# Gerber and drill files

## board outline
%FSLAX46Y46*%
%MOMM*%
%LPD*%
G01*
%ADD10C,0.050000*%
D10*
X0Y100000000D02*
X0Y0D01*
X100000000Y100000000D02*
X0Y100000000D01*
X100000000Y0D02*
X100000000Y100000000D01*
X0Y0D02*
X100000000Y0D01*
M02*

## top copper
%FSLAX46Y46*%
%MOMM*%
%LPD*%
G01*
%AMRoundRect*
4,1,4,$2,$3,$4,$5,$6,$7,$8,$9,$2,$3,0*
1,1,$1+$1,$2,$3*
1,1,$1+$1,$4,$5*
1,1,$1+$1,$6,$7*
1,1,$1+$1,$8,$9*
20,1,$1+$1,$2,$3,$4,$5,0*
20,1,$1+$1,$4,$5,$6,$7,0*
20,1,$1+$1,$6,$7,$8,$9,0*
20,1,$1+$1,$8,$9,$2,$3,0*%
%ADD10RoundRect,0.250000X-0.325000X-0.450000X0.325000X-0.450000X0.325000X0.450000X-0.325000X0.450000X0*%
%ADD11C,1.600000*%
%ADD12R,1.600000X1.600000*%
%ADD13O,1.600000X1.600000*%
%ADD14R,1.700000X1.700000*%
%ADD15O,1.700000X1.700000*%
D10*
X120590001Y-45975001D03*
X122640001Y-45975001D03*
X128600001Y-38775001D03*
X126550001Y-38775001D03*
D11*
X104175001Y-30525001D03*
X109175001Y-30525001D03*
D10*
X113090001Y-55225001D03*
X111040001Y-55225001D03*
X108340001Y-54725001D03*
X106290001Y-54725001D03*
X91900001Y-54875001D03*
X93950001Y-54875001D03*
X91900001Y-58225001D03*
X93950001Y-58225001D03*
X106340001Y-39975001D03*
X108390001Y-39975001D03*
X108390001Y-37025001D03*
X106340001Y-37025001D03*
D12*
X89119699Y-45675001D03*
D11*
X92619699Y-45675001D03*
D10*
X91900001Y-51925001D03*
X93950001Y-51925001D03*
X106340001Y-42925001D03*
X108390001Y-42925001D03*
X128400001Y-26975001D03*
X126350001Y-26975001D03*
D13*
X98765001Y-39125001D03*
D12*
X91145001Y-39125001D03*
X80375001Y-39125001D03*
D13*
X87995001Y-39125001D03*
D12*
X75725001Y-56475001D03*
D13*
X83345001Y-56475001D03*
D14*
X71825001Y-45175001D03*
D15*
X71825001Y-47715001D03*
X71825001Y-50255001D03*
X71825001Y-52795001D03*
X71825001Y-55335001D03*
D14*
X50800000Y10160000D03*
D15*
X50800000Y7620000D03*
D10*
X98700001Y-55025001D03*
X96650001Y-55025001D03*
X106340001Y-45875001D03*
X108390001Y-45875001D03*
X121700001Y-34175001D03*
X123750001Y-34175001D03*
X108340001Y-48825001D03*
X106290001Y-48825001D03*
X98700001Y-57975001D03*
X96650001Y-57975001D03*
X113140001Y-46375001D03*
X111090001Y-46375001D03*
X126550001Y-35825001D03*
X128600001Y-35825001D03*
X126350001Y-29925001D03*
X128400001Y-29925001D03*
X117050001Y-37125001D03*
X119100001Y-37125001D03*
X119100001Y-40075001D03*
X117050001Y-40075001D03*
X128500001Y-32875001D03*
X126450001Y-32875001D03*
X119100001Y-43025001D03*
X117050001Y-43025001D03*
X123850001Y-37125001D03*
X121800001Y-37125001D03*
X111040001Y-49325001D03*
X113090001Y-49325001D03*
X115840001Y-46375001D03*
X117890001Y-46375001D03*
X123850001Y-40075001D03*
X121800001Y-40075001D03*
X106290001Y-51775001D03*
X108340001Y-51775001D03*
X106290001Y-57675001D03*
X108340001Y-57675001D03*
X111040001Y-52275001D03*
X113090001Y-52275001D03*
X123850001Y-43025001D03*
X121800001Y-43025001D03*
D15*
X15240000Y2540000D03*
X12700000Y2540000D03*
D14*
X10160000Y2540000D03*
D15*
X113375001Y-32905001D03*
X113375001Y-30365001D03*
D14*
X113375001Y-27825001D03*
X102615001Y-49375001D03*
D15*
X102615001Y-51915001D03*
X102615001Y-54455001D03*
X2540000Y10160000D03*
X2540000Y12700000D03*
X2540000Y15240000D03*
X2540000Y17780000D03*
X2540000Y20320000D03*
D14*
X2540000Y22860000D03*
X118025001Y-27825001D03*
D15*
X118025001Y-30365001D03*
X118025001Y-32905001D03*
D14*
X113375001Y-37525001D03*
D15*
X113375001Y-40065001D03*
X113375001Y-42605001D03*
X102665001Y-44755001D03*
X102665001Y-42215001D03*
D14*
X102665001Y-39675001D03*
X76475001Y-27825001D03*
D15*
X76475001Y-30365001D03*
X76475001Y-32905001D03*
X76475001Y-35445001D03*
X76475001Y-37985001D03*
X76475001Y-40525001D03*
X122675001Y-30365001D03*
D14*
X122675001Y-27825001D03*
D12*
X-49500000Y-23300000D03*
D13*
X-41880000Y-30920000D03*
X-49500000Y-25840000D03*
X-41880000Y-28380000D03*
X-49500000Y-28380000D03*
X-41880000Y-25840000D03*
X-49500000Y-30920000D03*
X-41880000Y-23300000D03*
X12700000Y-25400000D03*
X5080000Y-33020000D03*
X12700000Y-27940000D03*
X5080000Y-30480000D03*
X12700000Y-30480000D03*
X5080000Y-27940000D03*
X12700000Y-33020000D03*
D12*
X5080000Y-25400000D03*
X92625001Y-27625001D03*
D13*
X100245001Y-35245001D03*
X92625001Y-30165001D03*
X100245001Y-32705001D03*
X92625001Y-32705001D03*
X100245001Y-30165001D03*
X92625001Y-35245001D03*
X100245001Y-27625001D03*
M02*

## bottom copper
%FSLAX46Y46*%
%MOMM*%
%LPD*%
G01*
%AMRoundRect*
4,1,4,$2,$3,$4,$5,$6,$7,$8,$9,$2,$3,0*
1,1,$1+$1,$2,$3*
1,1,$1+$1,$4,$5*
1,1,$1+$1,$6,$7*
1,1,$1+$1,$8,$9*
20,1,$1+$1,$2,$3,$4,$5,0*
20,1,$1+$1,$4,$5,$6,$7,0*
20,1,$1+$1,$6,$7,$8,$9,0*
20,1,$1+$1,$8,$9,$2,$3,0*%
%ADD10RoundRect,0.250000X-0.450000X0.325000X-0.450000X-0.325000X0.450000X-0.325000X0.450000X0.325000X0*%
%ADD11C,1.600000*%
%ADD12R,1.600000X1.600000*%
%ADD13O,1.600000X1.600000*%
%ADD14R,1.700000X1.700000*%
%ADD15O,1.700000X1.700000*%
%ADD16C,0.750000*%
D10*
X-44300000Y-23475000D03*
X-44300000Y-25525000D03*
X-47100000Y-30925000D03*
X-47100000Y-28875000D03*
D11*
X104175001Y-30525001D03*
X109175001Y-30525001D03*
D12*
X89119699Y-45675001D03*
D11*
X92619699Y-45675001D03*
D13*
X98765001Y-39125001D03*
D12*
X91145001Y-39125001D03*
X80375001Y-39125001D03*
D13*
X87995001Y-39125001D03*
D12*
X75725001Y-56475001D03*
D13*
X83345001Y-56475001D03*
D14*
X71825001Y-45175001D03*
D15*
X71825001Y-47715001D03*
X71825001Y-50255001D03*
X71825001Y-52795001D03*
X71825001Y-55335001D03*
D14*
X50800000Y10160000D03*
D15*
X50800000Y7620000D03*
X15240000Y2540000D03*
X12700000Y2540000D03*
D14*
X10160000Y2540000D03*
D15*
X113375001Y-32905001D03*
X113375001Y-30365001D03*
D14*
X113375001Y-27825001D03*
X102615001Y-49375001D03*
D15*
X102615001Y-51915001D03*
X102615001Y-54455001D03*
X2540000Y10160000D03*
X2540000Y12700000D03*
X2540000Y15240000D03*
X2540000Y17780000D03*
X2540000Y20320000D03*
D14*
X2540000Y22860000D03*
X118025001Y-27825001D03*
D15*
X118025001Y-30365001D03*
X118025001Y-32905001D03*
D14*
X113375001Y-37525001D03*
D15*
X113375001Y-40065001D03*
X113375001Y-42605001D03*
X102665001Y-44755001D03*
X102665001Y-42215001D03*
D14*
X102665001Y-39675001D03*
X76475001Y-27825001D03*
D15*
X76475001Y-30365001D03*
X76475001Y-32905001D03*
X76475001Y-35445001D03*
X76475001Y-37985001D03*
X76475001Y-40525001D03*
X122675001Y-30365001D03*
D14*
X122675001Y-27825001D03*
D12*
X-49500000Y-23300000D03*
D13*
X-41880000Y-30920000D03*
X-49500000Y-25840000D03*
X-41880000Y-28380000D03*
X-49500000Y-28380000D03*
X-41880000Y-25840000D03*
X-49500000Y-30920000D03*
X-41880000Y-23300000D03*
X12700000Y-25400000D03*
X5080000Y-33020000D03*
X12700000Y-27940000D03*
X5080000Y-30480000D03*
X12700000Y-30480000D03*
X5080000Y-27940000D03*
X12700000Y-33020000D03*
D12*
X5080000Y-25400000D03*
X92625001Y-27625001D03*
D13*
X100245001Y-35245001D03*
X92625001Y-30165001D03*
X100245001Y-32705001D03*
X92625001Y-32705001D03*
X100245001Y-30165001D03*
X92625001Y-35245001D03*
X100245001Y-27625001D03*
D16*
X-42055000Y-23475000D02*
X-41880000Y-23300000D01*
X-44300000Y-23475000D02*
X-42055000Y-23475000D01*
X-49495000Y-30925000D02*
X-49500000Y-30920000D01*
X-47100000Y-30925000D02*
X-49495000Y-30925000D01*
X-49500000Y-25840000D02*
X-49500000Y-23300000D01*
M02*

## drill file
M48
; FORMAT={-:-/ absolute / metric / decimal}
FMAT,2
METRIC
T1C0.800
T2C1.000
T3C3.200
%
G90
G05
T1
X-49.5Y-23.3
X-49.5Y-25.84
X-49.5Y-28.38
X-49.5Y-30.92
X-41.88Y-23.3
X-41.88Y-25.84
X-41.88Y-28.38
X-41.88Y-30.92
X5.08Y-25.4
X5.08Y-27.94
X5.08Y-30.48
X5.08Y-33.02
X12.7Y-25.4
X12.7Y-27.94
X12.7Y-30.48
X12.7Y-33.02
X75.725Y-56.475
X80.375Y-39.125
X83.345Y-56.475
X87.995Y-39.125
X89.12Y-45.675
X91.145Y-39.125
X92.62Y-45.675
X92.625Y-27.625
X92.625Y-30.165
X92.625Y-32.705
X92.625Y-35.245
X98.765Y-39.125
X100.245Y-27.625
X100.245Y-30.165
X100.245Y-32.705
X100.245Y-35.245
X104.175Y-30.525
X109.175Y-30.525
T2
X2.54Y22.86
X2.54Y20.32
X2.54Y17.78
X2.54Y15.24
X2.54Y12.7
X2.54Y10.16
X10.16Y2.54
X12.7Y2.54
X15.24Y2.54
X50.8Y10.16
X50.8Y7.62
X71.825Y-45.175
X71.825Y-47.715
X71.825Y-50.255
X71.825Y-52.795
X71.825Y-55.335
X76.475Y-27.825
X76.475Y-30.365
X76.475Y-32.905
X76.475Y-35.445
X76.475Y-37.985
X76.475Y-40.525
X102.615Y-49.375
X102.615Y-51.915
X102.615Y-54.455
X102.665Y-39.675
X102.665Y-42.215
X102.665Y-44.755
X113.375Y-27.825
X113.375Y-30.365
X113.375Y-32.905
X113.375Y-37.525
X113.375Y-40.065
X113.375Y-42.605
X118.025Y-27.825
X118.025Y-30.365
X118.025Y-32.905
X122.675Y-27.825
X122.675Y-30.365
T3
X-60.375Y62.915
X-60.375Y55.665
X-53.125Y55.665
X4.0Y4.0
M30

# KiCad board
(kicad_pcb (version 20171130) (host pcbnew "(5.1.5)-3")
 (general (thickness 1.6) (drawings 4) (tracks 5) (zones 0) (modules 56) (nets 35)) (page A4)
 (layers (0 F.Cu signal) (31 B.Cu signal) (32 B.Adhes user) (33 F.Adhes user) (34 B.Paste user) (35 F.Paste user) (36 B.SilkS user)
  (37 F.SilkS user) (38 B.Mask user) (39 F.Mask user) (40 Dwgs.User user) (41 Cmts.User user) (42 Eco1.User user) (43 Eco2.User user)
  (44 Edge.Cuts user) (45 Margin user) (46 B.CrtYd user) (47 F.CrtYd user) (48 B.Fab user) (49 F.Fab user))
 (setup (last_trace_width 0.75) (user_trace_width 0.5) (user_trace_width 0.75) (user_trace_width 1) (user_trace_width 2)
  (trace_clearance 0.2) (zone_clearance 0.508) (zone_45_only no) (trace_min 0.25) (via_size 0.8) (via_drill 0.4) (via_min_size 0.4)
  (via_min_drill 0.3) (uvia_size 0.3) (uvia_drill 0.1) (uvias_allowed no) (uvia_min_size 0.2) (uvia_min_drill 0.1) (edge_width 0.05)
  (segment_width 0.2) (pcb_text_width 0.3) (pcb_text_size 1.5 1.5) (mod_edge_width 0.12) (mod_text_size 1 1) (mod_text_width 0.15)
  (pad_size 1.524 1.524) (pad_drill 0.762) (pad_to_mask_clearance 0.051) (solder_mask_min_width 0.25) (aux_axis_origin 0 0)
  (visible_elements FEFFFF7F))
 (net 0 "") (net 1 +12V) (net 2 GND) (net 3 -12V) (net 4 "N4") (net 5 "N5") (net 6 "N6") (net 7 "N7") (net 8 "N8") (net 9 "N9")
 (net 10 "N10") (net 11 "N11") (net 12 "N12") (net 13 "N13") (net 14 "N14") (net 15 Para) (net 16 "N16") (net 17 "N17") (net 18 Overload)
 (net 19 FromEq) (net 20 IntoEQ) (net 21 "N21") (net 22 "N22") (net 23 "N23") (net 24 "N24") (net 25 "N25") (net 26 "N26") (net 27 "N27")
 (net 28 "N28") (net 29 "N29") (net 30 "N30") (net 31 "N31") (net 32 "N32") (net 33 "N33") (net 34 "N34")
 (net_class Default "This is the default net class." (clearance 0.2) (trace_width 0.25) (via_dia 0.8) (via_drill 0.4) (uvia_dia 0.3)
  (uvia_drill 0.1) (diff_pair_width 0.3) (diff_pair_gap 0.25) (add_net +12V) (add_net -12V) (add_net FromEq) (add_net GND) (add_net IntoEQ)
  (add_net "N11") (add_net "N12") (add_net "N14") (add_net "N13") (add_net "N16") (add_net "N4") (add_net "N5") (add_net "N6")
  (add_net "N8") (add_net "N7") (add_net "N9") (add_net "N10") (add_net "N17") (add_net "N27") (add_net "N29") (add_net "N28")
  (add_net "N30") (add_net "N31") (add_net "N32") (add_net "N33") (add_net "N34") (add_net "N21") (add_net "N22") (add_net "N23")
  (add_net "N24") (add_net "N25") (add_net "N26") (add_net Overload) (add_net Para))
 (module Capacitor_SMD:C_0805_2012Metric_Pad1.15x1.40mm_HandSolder (layer B.Cu) (at -44.3 24.5 270)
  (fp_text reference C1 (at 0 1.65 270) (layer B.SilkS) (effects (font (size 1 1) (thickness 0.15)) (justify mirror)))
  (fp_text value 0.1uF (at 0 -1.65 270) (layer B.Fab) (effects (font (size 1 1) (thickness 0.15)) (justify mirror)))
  (pad 1 smd roundrect (at -1.025 0 270) (size 1.15 1.4) (layers B.Cu B.Paste B.Mask) (roundrect_rratio 0.217391) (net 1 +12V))
  (pad 2 smd roundrect (at 1.025 0 270) (size 1.15 1.4) (layers B.Cu B.Paste B.Mask) (roundrect_rratio 0.217391) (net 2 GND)))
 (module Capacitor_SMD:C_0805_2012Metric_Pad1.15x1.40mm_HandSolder (layer B.Cu) (at -47.1 29.9 270)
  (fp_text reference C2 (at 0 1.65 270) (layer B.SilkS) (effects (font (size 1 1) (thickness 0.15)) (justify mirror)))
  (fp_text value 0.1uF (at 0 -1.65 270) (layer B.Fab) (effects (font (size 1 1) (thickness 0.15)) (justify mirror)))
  (pad 2 smd roundrect (at 1.025 0 270) (size 1.15 1.4) (layers B.Cu B.Paste B.Mask) (roundrect_rratio 0.217391) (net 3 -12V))
  (pad 1 smd roundrect (at -1.025 0 270) (size 1.15 1.4) (layers B.Cu B.Paste B.Mask) (roundrect_rratio 0.217391) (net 2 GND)))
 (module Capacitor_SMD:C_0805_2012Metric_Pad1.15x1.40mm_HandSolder (layer F.Cu) (at 121.615001 45.975001)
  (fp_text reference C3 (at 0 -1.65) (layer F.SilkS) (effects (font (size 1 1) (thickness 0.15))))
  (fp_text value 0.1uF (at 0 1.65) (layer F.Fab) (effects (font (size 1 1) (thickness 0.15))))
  (pad 1 smd roundrect (at -1.025 0) (size 1.15 1.4) (layers F.Cu F.Paste F.Mask) (roundrect_rratio 0.217391) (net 1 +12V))
  (pad 2 smd roundrect (at 1.025 0) (size 1.15 1.4) (layers F.Cu F.Paste F.Mask) (roundrect_rratio 0.217391) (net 2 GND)))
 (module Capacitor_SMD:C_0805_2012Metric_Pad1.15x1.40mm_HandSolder (layer F.Cu) (at 127.575001 38.775001)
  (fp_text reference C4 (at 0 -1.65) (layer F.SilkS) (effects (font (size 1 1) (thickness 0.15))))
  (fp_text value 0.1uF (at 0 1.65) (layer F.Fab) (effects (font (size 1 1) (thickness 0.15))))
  (pad 2 smd roundrect (at 1.025 0) (size 1.15 1.4) (layers F.Cu F.Paste F.Mask) (roundrect_rratio 0.217391) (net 3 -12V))
  (pad 1 smd roundrect (at -1.025 0) (size 1.15 1.4) (layers F.Cu F.Paste F.Mask) (roundrect_rratio 0.217391) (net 2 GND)))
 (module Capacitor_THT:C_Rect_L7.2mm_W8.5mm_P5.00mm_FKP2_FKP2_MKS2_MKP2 (layer F.Cu) (at 104.175001 30.525001)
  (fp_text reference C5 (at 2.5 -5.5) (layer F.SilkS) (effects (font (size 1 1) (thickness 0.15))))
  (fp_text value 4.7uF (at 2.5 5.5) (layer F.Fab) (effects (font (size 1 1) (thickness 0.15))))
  (pad 1 thru_hole circle (at 0 0) (size 1.6 1.6) (drill 0.8) (layers *.Cu *.Mask) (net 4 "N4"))
  (pad 2 thru_hole circle (at 5 0) (size 1.6 1.6) (drill 0.8) (layers *.Cu *.Mask) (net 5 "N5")))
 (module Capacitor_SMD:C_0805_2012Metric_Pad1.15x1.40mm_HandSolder (layer F.Cu) (at 112.065001 55.225001)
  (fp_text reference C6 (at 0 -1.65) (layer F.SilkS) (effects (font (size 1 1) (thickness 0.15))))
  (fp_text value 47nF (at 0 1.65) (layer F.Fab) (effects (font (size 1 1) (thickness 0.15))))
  (pad 2 smd roundrect (at 1.025 0) (size 1.15 1.4) (layers F.Cu F.Paste F.Mask) (roundrect_rratio 0.217391) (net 4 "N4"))
  (pad 1 smd roundrect (at -1.025 0) (size 1.15 1.4) (layers F.Cu F.Paste F.Mask) (roundrect_rratio 0.217391) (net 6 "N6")))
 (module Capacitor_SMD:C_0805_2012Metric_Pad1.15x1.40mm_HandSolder (layer F.Cu) (at 107.315001 54.725001)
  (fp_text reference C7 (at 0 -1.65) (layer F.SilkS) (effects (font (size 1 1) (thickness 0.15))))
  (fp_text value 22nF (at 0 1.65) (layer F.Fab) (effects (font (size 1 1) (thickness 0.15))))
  (pad 2 smd roundrect (at 1.025 0) (size 1.15 1.4) (layers F.Cu F.Paste F.Mask) (roundrect_rratio 0.217391) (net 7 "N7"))
  (pad 1 smd roundrect (at -1.025 0) (size 1.15 1.4) (layers F.Cu F.Paste F.Mask) (roundrect_rratio 0.217391) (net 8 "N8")))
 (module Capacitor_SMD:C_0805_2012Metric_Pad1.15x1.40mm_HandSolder (layer F.Cu) (at 92.925001 54.875001)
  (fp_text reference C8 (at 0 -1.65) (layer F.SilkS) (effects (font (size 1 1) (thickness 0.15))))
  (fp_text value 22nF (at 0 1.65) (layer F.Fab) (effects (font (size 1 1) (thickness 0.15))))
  (pad 1 smd roundrect (at -1.025 0) (size 1.15 1.4) (layers F.Cu F.Paste F.Mask) (roundrect_rratio 0.217391) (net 2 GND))
  (pad 2 smd roundrect (at 1.025 0) (size 1.15 1.4) (layers F.Cu F.Paste F.Mask) (roundrect_rratio 0.217391) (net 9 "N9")))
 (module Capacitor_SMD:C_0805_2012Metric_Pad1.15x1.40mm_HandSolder (layer F.Cu) (at 92.925001 58.225001)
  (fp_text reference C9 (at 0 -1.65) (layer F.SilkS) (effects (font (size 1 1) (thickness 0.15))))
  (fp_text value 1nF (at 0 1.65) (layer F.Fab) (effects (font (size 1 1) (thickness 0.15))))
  (pad 1 smd roundrect (at -1.025 0) (size 1.15 1.4) (layers F.Cu F.Paste F.Mask) (roundrect_rratio 0.217391) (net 2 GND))
  (pad 2 smd roundrect (at 1.025 0) (size 1.15 1.4) (layers F.Cu F.Paste F.Mask) (roundrect_rratio 0.217391) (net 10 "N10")))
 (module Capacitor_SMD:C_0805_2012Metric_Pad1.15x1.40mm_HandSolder (layer F.Cu) (at 107.365001 39.975001)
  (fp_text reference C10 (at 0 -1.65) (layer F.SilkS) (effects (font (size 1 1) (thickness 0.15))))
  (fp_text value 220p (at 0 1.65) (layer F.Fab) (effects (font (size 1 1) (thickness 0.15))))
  (pad 1 smd roundrect (at -1.025 0) (size 1.15 1.4) (layers F.Cu F.Paste F.Mask) (roundrect_rratio 0.217391) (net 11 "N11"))
  (pad 2 smd roundrect (at 1.025 0) (size 1.15 1.4) (layers F.Cu F.Paste F.Mask) (roundrect_rratio 0.217391) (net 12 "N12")))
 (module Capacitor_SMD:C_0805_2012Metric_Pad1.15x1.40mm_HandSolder (layer F.Cu) (at 107.365001 37.025001)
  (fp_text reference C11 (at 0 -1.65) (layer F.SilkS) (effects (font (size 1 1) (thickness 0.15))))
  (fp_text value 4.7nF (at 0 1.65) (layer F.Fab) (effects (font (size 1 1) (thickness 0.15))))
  (pad 2 smd roundrect (at 1.025 0) (size 1.15 1.4) (layers F.Cu F.Paste F.Mask) (roundrect_rratio 0.217391) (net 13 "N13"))
  (pad 1 smd roundrect (at -1.025 0) (size 1.15 1.4) (layers F.Cu F.Paste F.Mask) (roundrect_rratio 0.217391) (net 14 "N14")))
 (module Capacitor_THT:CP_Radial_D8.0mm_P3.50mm (layer F.Cu) (at 89.119699 45.675001)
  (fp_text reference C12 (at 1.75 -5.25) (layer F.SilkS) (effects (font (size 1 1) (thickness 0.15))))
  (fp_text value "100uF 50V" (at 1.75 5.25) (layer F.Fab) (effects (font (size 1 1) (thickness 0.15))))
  (pad 1 thru_hole rect (at 0 0) (size 1.6 1.6) (drill 0.8) (layers *.Cu *.Mask) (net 11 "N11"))
  (pad 2 thru_hole circle (at 3.5 0) (size 1.6 1.6) (drill 0.8) (layers *.Cu *.Mask) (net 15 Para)))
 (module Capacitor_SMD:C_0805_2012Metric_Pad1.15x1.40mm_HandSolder (layer F.Cu) (at 92.925001 51.925001)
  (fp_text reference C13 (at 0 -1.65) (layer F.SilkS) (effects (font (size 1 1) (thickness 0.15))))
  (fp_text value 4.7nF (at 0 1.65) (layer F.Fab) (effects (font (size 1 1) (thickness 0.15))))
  (pad 1 smd roundrect (at -1.025 0) (size 1.15 1.4) (layers F.Cu F.Paste F.Mask) (roundrect_rratio 0.217391) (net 2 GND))
  (pad 2 smd roundrect (at 1.025 0) (size 1.15 1.4) (layers F.Cu F.Paste F.Mask) (roundrect_rratio 0.217391) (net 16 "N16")))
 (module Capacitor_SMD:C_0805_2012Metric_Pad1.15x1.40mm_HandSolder (layer F.Cu) (at 107.365001 42.925001)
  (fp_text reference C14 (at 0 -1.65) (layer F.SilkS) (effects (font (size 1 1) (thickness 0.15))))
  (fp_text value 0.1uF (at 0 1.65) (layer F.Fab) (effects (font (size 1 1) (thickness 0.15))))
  (pad 1 smd roundrect (at -1.025 0) (size 1.15 1.4) (layers F.Cu F.Paste F.Mask) (roundrect_rratio 0.217391) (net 1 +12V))
  (pad 2 smd roundrect (at 1.025 0) (size 1.15 1.4) (layers F.Cu F.Paste F.Mask) (roundrect_rratio 0.217391) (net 2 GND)))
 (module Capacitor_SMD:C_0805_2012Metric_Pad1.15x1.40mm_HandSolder (layer F.Cu) (at 127.375001 26.975001)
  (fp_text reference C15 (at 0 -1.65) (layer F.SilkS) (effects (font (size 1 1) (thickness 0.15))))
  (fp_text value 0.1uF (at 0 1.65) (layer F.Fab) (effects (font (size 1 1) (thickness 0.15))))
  (pad 2 smd roundrect (at 1.025 0) (size 1.15 1.4) (layers F.Cu F.Paste F.Mask) (roundrect_rratio 0.217391) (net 3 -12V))
  (pad 1 smd roundrect (at -1.025 0) (size 1.15 1.4) (layers F.Cu F.Paste F.Mask) (roundrect_rratio 0.217391) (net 2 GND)))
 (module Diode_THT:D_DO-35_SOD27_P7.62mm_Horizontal (layer F.Cu) (at 91.145001 39.125001)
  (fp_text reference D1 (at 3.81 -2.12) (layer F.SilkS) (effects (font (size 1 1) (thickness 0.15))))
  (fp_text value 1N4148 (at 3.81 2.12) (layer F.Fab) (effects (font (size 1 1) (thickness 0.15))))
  (pad 2 thru_hole oval (at 7.62 0) (size 1.6 1.6) (drill 0.8) (layers *.Cu *.Mask) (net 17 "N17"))
  (pad 1 thru_hole rect (at 0 0) (size 1.6 1.6) (drill 0.8) (layers *.Cu *.Mask) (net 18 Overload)))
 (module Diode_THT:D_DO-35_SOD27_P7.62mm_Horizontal (layer F.Cu) (at 80.375001 39.125001)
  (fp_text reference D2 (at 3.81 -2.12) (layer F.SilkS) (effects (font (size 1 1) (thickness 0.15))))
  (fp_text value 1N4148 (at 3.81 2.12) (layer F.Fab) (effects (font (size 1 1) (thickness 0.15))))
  (pad 1 thru_hole rect (at 0 0) (size 1.6 1.6) (drill 0.8) (layers *.Cu *.Mask) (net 18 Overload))
  (pad 2 thru_hole oval (at 7.62 0) (size 1.6 1.6) (drill 0.8) (layers *.Cu *.Mask) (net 11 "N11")))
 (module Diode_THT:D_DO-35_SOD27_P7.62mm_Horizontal (layer F.Cu) (at 75.725001 56.475001)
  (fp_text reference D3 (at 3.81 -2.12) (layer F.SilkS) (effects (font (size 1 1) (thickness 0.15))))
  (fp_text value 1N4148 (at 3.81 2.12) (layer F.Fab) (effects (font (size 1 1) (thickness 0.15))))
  (pad 1 thru_hole rect (at 0 0) (size 1.6 1.6) (drill 0.8) (layers *.Cu *.Mask) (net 18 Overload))
  (pad 2 thru_hole oval (at 7.62 0) (size 1.6 1.6) (drill 0.8) (layers *.Cu *.Mask) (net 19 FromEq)))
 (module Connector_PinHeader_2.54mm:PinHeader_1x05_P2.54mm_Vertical (layer F.Cu) (at 71.825001 45.175001)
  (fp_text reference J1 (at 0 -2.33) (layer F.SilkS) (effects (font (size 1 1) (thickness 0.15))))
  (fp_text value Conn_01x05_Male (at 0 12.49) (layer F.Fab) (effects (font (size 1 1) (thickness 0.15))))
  (pad 1 thru_hole rect (at 0 0) (size 1.7 1.7) (drill 1) (layers *.Cu *.Mask) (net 1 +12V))
  (pad 2 thru_hole oval (at 0 2.54) (size 1.7 1.7) (drill 1) (layers *.Cu *.Mask) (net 3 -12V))
  (pad 3 thru_hole oval (at 0 5.08) (size 1.7 1.7) (drill 1) (layers *.Cu *.Mask) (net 2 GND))
  (pad 4 thru_hole oval (at 0 7.62) (size 1.7 1.7) (drill 1) (layers *.Cu *.Mask) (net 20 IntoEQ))
  (pad 5 thru_hole oval (at 0 10.16) (size 1.7 1.7) (drill 1) (layers *.Cu *.Mask) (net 19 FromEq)))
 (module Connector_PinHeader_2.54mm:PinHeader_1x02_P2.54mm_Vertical (layer F.Cu) (at 50.8 -10.16)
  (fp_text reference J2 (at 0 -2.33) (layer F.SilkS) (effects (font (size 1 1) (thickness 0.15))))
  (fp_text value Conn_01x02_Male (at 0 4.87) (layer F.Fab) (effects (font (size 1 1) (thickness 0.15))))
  (pad 1 thru_hole rect (at 0 0) (size 1.7 1.7) (drill 1) (layers *.Cu *.Mask) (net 2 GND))
  (pad 2 thru_hole oval (at 0 2.54) (size 1.7 1.7) (drill 1) (layers *.Cu *.Mask) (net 18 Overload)))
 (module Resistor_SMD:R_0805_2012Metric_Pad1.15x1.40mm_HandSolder (layer F.Cu) (at 97.675001 55.025001)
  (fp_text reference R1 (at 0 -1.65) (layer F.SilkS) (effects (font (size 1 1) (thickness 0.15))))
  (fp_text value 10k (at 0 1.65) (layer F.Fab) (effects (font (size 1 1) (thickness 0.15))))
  (pad 2 smd roundrect (at 1.025 0) (size 1.15 1.4) (layers F.Cu F.Paste F.Mask) (roundrect_rratio 0.217391) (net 2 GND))
  (pad 1 smd roundrect (at -1.025 0) (size 1.15 1.4) (layers F.Cu F.Paste F.Mask) (roundrect_rratio 0.217391) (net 20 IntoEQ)))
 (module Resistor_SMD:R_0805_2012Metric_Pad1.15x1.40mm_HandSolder (layer F.Cu) (at 107.365001 45.875001)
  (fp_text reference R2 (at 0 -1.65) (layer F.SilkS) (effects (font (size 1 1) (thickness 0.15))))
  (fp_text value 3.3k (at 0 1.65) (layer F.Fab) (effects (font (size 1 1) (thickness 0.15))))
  (pad 1 smd roundrect (at -1.025 0) (size 1.15 1.4) (layers F.Cu F.Paste F.Mask) (roundrect_rratio 0.217391) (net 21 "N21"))
  (pad 2 smd roundrect (at 1.025 0) (size 1.15 1.4) (layers F.Cu F.Paste F.Mask) (roundrect_rratio 0.217391) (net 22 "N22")))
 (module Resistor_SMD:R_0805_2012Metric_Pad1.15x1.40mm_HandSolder (layer F.Cu) (at 122.725001 34.175001)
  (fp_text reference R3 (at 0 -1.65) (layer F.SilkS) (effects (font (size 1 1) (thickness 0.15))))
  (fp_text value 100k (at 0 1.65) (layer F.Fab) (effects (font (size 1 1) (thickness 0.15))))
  (pad 1 smd roundrect (at -1.025 0) (size 1.15 1.4) (layers F.Cu F.Paste F.Mask) (roundrect_rratio 0.217391) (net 15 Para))
  (pad 2 smd roundrect (at 1.025 0) (size 1.15 1.4) (layers F.Cu F.Paste F.Mask) (roundrect_rratio 0.217391) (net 2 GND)))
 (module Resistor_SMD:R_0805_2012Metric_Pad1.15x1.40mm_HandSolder (layer F.Cu) (at 107.315001 48.825001)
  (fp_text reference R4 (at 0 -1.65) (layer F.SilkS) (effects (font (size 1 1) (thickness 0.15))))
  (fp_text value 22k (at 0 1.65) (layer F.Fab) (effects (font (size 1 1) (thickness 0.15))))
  (pad 2 smd roundrect (at 1.025 0) (size 1.15 1.4) (layers F.Cu F.Paste F.Mask) (roundrect_rratio 0.217391) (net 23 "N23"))
  (pad 1 smd roundrect (at -1.025 0) (size 1.15 1.4) (layers F.Cu F.Paste F.Mask) (roundrect_rratio 0.217391) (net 6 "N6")))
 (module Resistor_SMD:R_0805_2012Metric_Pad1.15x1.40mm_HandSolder (layer F.Cu) (at 97.675001 57.975001)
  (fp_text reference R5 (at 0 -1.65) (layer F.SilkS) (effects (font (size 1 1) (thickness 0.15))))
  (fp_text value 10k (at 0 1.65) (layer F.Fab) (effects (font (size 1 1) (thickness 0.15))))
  (pad 2 smd roundrect (at 1.025 0) (size 1.15 1.4) (layers F.Cu F.Paste F.Mask) (roundrect_rratio 0.217391) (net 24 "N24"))
  (pad 1 smd roundrect (at -1.025 0) (size 1.15 1.4) (layers F.Cu F.Paste F.Mask) (roundrect_rratio 0.217391) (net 8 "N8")))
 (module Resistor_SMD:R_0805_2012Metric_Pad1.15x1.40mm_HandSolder (layer F.Cu) (at 112.115001 46.375001)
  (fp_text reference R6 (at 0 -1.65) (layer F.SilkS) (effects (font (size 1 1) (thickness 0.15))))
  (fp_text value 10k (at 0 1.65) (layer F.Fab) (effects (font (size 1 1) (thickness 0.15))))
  (pad 2 smd roundrect (at 1.025 0) (size 1.15 1.4) (layers F.Cu F.Paste F.Mask) (roundrect_rratio 0.217391) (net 2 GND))
  (pad 1 smd roundrect (at -1.025 0) (size 1.15 1.4) (layers F.Cu F.Paste F.Mask) (roundrect_rratio 0.217391) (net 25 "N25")))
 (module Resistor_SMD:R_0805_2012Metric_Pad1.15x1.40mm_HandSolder (layer F.Cu) (at 127.575001 35.825001)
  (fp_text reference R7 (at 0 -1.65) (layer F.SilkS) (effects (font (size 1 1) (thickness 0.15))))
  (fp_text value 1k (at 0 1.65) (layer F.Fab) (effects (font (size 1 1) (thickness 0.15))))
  (pad 1 smd roundrect (at -1.025 0) (size 1.15 1.4) (layers F.Cu F.Paste F.Mask) (roundrect_rratio 0.217391) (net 4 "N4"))
  (pad 2 smd roundrect (at 1.025 0) (size 1.15 1.4) (layers F.Cu F.Paste F.Mask) (roundrect_rratio 0.217391) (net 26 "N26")))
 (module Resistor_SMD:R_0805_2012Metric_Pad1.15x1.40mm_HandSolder (layer F.Cu) (at 127.375001 29.925001)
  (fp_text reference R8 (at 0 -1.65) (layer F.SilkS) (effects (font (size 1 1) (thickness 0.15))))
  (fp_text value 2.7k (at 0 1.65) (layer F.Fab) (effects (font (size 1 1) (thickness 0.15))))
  (pad 1 smd roundrect (at -1.025 0) (size 1.15 1.4) (layers F.Cu F.Paste F.Mask) (roundrect_rratio 0.217391) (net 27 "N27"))
  (pad 2 smd roundrect (at 1.025 0) (size 1.15 1.4) (layers F.Cu F.Paste F.Mask) (roundrect_rratio 0.217391) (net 15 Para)))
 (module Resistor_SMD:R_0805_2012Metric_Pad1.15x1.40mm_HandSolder (layer F.Cu) (at 118.075001 37.125001)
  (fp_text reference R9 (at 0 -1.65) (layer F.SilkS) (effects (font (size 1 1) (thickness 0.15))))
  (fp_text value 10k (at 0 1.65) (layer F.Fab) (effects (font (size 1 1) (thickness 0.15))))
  (pad 1 smd roundrect (at -1.025 0) (size 1.15 1.4) (layers F.Cu F.Paste F.Mask) (roundrect_rratio 0.217391) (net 27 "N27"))
  (pad 2 smd roundrect (at 1.025 0) (size 1.15 1.4) (layers F.Cu F.Paste F.Mask) (roundrect_rratio 0.217391) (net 2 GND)))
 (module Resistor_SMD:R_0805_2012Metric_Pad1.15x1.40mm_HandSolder (layer F.Cu) (at 118.075001 40.075001)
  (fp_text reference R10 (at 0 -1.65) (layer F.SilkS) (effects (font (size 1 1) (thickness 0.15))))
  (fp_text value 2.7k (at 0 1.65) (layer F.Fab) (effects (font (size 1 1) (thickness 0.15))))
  (pad 2 smd roundrect (at 1.025 0) (size 1.15 1.4) (layers F.Cu F.Paste F.Mask) (roundrect_rratio 0.217391) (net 27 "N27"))
  (pad 1 smd roundrect (at -1.025 0) (size 1.15 1.4) (layers F.Cu F.Paste F.Mask) (roundrect_rratio 0.217391) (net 17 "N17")))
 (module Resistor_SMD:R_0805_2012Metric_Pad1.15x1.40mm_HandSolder (layer F.Cu) (at 127.475001 32.875001)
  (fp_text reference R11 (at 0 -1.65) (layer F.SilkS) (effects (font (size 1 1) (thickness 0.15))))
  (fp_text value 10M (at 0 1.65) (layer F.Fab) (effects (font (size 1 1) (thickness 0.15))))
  (pad 2 smd roundrect (at 1.025 0) (size 1.15 1.4) (layers F.Cu F.Paste F.Mask) (roundrect_rratio 0.217391) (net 2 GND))
  (pad 1 smd roundrect (at -1.025 0) (size 1.15 1.4) (layers F.Cu F.Paste F.Mask) (roundrect_rratio 0.217391) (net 10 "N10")))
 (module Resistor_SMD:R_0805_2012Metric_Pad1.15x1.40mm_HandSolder (layer F.Cu) (at 118.075001 43.025001)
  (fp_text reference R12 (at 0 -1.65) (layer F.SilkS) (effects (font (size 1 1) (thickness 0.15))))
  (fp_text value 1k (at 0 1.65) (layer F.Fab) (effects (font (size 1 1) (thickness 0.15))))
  (pad 2 smd roundrect (at 1.025 0) (size 1.15 1.4) (layers F.Cu F.Paste F.Mask) (roundrect_rratio 0.217391) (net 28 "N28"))
  (pad 1 smd roundrect (at -1.025 0) (size 1.15 1.4) (layers F.Cu F.Paste F.Mask) (roundrect_rratio 0.217391) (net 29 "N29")))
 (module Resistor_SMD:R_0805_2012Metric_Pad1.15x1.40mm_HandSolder (layer F.Cu) (at 122.825001 37.125001)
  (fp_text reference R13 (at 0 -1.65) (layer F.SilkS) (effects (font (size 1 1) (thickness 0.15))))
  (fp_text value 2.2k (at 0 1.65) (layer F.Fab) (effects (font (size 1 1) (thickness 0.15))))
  (pad 2 smd roundrect (at 1.025 0) (size 1.15 1.4) (layers F.Cu F.Paste F.Mask) (roundrect_rratio 0.217391) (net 29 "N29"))
  (pad 1 smd roundrect (at -1.025 0) (size 1.15 1.4) (layers F.Cu F.Paste F.Mask) (roundrect_rratio 0.217391) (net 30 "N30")))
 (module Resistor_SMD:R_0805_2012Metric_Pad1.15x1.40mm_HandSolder (layer F.Cu) (at 112.065001 49.325001)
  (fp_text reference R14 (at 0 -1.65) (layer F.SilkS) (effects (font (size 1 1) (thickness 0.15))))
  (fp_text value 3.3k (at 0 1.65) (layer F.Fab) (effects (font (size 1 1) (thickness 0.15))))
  (pad 1 smd roundrect (at -1.025 0) (size 1.15 1.4) (layers F.Cu F.Paste F.Mask) (roundrect_rratio 0.217391) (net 11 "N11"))
  (pad 2 smd roundrect (at 1.025 0) (size 1.15 1.4) (layers F.Cu F.Paste F.Mask) (roundrect_rratio 0.217391) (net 12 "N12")))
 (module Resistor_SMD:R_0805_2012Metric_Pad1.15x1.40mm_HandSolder (layer F.Cu) (at 116.865001 46.375001)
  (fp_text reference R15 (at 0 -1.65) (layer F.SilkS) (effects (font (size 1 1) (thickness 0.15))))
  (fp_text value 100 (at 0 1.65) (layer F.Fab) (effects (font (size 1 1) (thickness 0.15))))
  (pad 1 smd roundrect (at -1.025 0) (size 1.15 1.4) (layers F.Cu F.Paste F.Mask) (roundrect_rratio 0.217391) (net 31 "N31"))
  (pad 2 smd roundrect (at 1.025 0) (size 1.15 1.4) (layers F.Cu F.Paste F.Mask) (roundrect_rratio 0.217391) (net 29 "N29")))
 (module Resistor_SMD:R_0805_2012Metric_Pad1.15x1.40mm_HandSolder (layer F.Cu) (at 122.825001 40.075001)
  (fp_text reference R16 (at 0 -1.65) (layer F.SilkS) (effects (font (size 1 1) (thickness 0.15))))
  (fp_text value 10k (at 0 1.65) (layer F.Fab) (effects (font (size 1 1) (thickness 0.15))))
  (pad 2 smd roundrect (at 1.025 0) (size 1.15 1.4) (layers F.Cu F.Paste F.Mask) (roundrect_rratio 0.217391) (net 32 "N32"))
  (pad 1 smd roundrect (at -1.025 0) (size 1.15 1.4) (layers F.Cu F.Paste F.Mask) (roundrect_rratio 0.217391) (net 14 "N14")))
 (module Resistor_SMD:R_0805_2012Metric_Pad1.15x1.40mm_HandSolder (layer F.Cu) (at 107.315001 51.775001)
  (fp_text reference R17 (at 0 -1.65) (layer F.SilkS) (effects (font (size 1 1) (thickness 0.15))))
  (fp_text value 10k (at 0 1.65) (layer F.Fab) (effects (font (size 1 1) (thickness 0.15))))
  (pad 1 smd roundrect (at -1.025 0) (size 1.15 1.4) (layers F.Cu F.Paste F.Mask) (roundrect_rratio 0.217391) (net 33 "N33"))
  (pad 2 smd roundrect (at 1.025 0) (size 1.15 1.4) (layers F.Cu F.Paste F.Mask) (roundrect_rratio 0.217391) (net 2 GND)))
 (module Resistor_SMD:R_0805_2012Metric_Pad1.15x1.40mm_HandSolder (layer F.Cu) (at 107.315001 57.675001)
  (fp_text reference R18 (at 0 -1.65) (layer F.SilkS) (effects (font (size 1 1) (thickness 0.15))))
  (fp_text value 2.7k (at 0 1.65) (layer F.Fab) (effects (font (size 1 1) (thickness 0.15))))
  (pad 1 smd roundrect (at -1.025 0) (size 1.15 1.4) (layers F.Cu F.Paste F.Mask) (roundrect_rratio 0.217391) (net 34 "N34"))
  (pad 2 smd roundrect (at 1.025 0) (size 1.15 1.4) (layers F.Cu F.Paste F.Mask) (roundrect_rratio 0.217391) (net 17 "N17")))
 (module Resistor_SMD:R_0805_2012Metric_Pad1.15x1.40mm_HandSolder (layer F.Cu) (at 112.065001 52.275001)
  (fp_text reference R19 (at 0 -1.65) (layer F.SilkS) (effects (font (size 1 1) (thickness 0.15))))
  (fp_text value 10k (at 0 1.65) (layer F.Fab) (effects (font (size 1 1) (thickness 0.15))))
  (pad 1 smd roundrect (at -1.025 0) (size 1.15 1.4) (layers F.Cu F.Paste F.Mask) (roundrect_rratio 0.217391) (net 34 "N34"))
  (pad 2 smd roundrect (at 1.025 0) (size 1.15 1.4) (layers F.Cu F.Paste F.Mask) (roundrect_rratio 0.217391) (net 2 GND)))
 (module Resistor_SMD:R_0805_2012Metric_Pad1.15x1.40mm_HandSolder (layer F.Cu) (at 122.825001 43.025001)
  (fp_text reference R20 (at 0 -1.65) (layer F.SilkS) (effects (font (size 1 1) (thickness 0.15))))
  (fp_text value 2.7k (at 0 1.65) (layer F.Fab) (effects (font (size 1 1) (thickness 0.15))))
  (pad 2 smd roundrect (at 1.025 0) (size 1.15 1.4) (layers F.Cu F.Paste F.Mask) (roundrect_rratio 0.217391) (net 34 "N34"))
  (pad 1 smd roundrect (at -1.025 0) (size 1.15 1.4) (layers F.Cu F.Paste F.Mask) (roundrect_rratio 0.217391) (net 19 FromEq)))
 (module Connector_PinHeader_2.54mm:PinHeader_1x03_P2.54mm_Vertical (layer F.Cu) (at 10.16 -2.54 90)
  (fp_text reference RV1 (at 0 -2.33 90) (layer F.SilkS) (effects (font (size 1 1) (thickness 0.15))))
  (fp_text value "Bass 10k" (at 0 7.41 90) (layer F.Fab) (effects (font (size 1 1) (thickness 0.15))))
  (pad 3 thru_hole oval (at 0 5.08 90) (size 1.7 1.7) (drill 1) (layers *.Cu *.Mask) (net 21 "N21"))
  (pad 2 thru_hole oval (at 0 2.54 90) (size 1.7 1.7) (drill 1) (layers *.Cu *.Mask) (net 5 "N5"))
  (pad 1 thru_hole rect (at 0 0 90) (size 1.7 1.7) (drill 1) (layers *.Cu *.Mask) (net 12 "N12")))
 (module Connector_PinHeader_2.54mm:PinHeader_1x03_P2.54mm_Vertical (layer F.Cu) (at 113.375001 27.825001)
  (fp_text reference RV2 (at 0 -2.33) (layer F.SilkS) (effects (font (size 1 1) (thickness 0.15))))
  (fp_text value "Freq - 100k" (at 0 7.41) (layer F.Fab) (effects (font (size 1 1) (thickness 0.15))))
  (pad 3 thru_hole oval (at 0 5.08) (size 1.7 1.7) (drill 1) (layers *.Cu *.Mask) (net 2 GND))
  (pad 2 thru_hole oval (at 0 2.54) (size 1.7 1.7) (drill 1) (layers *.Cu *.Mask) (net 2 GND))
  (pad 1 thru_hole rect (at 0 0) (size 1.7 1.7) (drill 1) (layers *.Cu *.Mask) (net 23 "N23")))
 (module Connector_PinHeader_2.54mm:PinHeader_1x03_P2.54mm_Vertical (layer F.Cu) (at 102.615001 49.375001)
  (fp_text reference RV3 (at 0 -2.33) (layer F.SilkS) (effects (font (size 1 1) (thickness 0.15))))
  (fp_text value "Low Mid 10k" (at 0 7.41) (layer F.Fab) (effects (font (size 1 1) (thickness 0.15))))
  (pad 1 thru_hole rect (at 0 0) (size 1.7 1.7) (drill 1) (layers *.Cu *.Mask) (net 17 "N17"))
  (pad 2 thru_hole oval (at 0 2.54) (size 1.7 1.7) (drill 1) (layers *.Cu *.Mask) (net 7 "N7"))
  (pad 3 thru_hole oval (at 0 5.08) (size 1.7 1.7) (drill 1) (layers *.Cu *.Mask) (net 15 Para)))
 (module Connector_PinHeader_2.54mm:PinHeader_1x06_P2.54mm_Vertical (layer F.Cu) (at 2.54 -22.86)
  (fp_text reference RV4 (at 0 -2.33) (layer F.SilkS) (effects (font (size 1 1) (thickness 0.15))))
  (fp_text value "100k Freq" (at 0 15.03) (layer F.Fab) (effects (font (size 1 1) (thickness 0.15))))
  (pad 6 thru_hole oval (at 0 12.7) (size 1.7 1.7) (drill 1) (layers *.Cu *.Mask) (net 25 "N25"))
  (pad 5 thru_hole oval (at 0 10.16) (size 1.7 1.7) (drill 1) (layers *.Cu *.Mask) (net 25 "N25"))
  (pad 4 thru_hole oval (at 0 7.62) (size 1.7 1.7) (drill 1) (layers *.Cu *.Mask) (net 9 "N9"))
  (pad 3 thru_hole oval (at 0 5.08) (size 1.7 1.7) (drill 1) (layers *.Cu *.Mask) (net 9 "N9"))
  (pad 2 thru_hole oval (at 0 2.54) (size 1.7 1.7) (drill 1) (layers *.Cu *.Mask) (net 9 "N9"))
  (pad 1 thru_hole rect (at 0 0) (size 1.7 1.7) (drill 1) (layers *.Cu *.Mask) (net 24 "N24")))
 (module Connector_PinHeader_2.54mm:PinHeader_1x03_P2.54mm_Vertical (layer F.Cu) (at 118.025001 27.825001)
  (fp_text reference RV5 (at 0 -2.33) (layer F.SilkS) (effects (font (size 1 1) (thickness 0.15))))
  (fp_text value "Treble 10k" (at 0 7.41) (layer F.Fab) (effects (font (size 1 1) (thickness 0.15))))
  (pad 1 thru_hole rect (at 0 0) (size 1.7 1.7) (drill 1) (layers *.Cu *.Mask) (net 12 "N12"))
  (pad 2 thru_hole oval (at 0 2.54) (size 1.7 1.7) (drill 1) (layers *.Cu *.Mask) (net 28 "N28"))
  (pad 3 thru_hole oval (at 0 5.08) (size 1.7 1.7) (drill 1) (layers *.Cu *.Mask) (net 21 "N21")))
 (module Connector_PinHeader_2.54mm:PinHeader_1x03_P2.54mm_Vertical (layer F.Cu) (at 113.375001 37.525001)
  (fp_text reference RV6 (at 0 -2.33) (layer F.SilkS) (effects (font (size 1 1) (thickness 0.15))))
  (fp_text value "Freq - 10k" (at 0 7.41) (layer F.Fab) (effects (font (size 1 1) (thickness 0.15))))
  (pad 1 thru_hole rect (at 0 0) (size 1.7 1.7) (drill 1) (layers *.Cu *.Mask) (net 30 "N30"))
  (pad 2 thru_hole oval (at 0 2.54) (size 1.7 1.7) (drill 1) (layers *.Cu *.Mask) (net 10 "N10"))
  (pad 3 thru_hole oval (at 0 5.08) (size 1.7 1.7) (drill 1) (layers *.Cu *.Mask) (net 10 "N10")))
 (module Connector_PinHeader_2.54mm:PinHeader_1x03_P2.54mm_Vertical (layer F.Cu) (at 102.665001 39.675001)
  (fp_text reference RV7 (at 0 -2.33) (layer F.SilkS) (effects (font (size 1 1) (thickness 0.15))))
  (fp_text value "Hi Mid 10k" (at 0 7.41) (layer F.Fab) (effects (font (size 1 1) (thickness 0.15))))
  (pad 3 thru_hole oval (at 0 5.08) (size 1.7 1.7) (drill 1) (layers *.Cu *.Mask) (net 17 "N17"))
  (pad 2 thru_hole oval (at 0 2.54) (size 1.7 1.7) (drill 1) (layers *.Cu *.Mask) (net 13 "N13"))
  (pad 1 thru_hole rect (at 0 0) (size 1.7 1.7) (drill 1) (layers *.Cu *.Mask) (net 19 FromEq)))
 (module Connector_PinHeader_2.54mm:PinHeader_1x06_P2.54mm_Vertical (layer F.Cu) (at 76.475001 27.825001)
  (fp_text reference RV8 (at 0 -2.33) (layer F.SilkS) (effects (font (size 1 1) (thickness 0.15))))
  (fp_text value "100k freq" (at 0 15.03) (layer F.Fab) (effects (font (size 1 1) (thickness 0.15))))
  (pad 1 thru_hole rect (at 0 0) (size 1.7 1.7) (drill 1) (layers *.Cu *.Mask) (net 32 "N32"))
  (pad 2 thru_hole oval (at 0 2.54) (size 1.7 1.7) (drill 1) (layers *.Cu *.Mask) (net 16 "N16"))
  (pad 3 thru_hole oval (at 0 5.08) (size 1.7 1.7) (drill 1) (layers *.Cu *.Mask) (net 16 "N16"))
  (pad 4 thru_hole oval (at 0 7.62) (size 1.7 1.7) (drill 1) (layers *.Cu *.Mask) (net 16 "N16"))
  (pad 5 thru_hole oval (at 0 10.16) (size 1.7 1.7) (drill 1) (layers *.Cu *.Mask) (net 33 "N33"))
  (pad 6 thru_hole oval (at 0 12.7) (size 1.7 1.7) (drill 1) (layers *.Cu *.Mask) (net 33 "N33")))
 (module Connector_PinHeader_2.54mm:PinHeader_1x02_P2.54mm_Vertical (layer F.Cu) (at 122.675001 27.825001)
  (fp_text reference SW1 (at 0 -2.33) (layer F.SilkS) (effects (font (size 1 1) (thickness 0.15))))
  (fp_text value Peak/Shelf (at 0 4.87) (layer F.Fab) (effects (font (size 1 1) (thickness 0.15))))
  (pad 2 thru_hole oval (at 0 2.54) (size 1.7 1.7) (drill 1) (layers *.Cu *.Mask) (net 5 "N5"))
  (pad 1 thru_hole rect (at 0 0) (size 1.7 1.7) (drill 1) (layers *.Cu *.Mask) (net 4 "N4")))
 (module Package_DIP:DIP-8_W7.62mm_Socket (layer F.Cu) (at -49.5 23.3)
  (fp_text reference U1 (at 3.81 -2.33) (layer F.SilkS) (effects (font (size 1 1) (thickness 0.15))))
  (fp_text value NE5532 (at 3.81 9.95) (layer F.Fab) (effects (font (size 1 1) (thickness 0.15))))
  (pad 1 thru_hole rect (at 0 0) (size 1.6 1.6) (drill 0.8) (layers *.Cu *.Mask) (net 22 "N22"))
  (pad 5 thru_hole oval (at 7.62 7.62) (size 1.6 1.6) (drill 0.8) (layers *.Cu *.Mask) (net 21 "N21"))
  (pad 2 thru_hole oval (at 0 2.54) (size 1.6 1.6) (drill 0.8) (layers *.Cu *.Mask) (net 22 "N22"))
  (pad 6 thru_hole oval (at 7.62 5.08) (size 1.6 1.6) (drill 0.8) (layers *.Cu *.Mask) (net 12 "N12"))
  (pad 3 thru_hole oval (at 0 5.08) (size 1.6 1.6) (drill 0.8) (layers *.Cu *.Mask) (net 20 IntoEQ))
  (pad 7 thru_hole oval (at 7.62 2.54) (size 1.6 1.6) (drill 0.8) (layers *.Cu *.Mask) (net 11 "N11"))
  (pad 4 thru_hole oval (at 0 7.62) (size 1.6 1.6) (drill 0.8) (layers *.Cu *.Mask) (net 3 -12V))
  (pad 8 thru_hole oval (at 7.62 0) (size 1.6 1.6) (drill 0.8) (layers *.Cu *.Mask) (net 1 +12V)))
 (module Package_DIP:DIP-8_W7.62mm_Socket (layer F.Cu) (at 5.08 25.4)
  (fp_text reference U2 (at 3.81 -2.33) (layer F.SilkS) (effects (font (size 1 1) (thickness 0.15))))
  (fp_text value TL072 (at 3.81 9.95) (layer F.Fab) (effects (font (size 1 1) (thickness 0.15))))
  (pad 8 thru_hole oval (at 7.62 0) (size 1.6 1.6) (drill 0.8) (layers *.Cu *.Mask) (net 1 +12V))
  (pad 4 thru_hole oval (at 0 7.62) (size 1.6 1.6) (drill 0.8) (layers *.Cu *.Mask) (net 3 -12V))
  (pad 7 thru_hole oval (at 7.62 2.54) (size 1.6 1.6) (drill 0.8) (layers *.Cu *.Mask) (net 31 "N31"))
  (pad 3 thru_hole oval (at 0 5.08) (size 1.6 1.6) (drill 0.8) (layers *.Cu *.Mask) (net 6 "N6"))
  (pad 6 thru_hole oval (at 7.62 5.08) (size 1.6 1.6) (drill 0.8) (layers *.Cu *.Mask) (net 31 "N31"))
  (pad 2 thru_hole oval (at 0 2.54) (size 1.6 1.6) (drill 0.8) (layers *.Cu *.Mask) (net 26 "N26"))
  (pad 5 thru_hole oval (at 7.62 7.62) (size 1.6 1.6) (drill 0.8) (layers *.Cu *.Mask) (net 10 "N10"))
  (pad 1 thru_hole rect (at 0 0) (size 1.6 1.6) (drill 0.8) (layers *.Cu *.Mask) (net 26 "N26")))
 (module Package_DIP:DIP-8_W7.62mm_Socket (layer F.Cu) (at 92.625001 27.625001)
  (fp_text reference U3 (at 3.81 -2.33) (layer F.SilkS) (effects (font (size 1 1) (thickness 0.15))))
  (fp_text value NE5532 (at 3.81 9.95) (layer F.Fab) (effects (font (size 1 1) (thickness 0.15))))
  (pad 1 thru_hole rect (at 0 0) (size 1.6 1.6) (drill 0.8) (layers *.Cu *.Mask) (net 17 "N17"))
  (pad 5 thru_hole oval (at 7.62 7.62) (size 1.6 1.6) (drill 0.8) (layers *.Cu *.Mask) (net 16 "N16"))
  (pad 2 thru_hole oval (at 0 2.54) (size 1.6 1.6) (drill 0.8) (layers *.Cu *.Mask) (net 27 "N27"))
  (pad 6 thru_hole oval (at 7.62 5.08) (size 1.6 1.6) (drill 0.8) (layers *.Cu *.Mask) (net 34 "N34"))
  (pad 3 thru_hole oval (at 0 5.08) (size 1.6 1.6) (drill 0.8) (layers *.Cu *.Mask) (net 9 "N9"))
  (pad 7 thru_hole oval (at 7.62 2.54) (size 1.6 1.6) (drill 0.8) (layers *.Cu *.Mask) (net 19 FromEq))
  (pad 4 thru_hole oval (at 0 7.62) (size 1.6 1.6) (drill 0.8) (layers *.Cu *.Mask) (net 3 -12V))
  (pad 8 thru_hole oval (at 7.62 0) (size 1.6 1.6) (drill 0.8) (layers *.Cu *.Mask) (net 1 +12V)))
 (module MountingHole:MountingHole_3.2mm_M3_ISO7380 (layer F.Cu) (at -60.374999 -62.914999)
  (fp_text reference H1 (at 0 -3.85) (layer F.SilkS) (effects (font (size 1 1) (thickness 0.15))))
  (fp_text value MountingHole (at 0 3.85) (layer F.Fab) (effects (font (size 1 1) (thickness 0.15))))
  (pad 1 np_thru_hole circle (at 0 0) (size 3.2 3.2) (drill 3.2) (layers *.Cu *.Mask)))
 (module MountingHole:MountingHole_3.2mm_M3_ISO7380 (layer F.Cu) (at -60.374999 -55.664999)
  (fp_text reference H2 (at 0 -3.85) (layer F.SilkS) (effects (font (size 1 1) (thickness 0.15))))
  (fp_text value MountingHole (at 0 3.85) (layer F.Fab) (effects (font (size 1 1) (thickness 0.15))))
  (pad 1 np_thru_hole circle (at 0 0) (size 3.2 3.2) (drill 3.2) (layers *.Cu *.Mask)))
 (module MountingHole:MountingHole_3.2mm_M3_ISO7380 (layer F.Cu) (at 4 -4)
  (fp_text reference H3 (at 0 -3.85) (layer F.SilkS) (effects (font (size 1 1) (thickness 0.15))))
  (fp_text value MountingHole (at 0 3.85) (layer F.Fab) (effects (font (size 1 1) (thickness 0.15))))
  (pad 1 np_thru_hole circle (at 0 0) (size 3.2 3.2) (drill 3.2) (layers *.Cu *.Mask)))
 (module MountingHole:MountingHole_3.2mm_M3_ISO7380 (layer F.Cu) (at -53.124999 -55.664999)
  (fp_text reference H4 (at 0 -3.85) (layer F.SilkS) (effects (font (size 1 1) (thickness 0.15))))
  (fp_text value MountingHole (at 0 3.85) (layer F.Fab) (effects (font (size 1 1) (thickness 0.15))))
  (pad 1 np_thru_hole circle (at 0 0) (size 3.2 3.2) (drill 3.2) (layers *.Cu *.Mask)))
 (gr_line (start 0 -100) (end 0 0) (layer Edge.Cuts) (width 0.05))
 (gr_line (start 100 -100) (end 0 -100) (layer Edge.Cuts) (width 0.05))
 (gr_line (start 100 0) (end 100 -100) (layer Edge.Cuts) (width 0.05))
 (gr_line (start 0 0) (end 100 0) (layer Edge.Cuts) (width 0.05))
 (segment (start -42.055 23.475) (end -41.88 23.3) (width 0.75) (layer B.Cu) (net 1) (status 30))
 (segment (start -44.3 23.475) (end -42.055 23.475) (width 0.75) (layer B.Cu) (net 1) (status 30))
 (segment (start -49.495 30.925) (end -49.5 30.92) (width 0.75) (layer B.Cu) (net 3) (status 30))
 (segment (start -47.1 30.925) (end -49.495 30.925) (width 0.75) (layer B.Cu) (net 3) (status 30))
 (segment (start -49.5 25.84) (end -49.5 23.3) (width 0.75) (layer B.Cu) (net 22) (status 30)))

